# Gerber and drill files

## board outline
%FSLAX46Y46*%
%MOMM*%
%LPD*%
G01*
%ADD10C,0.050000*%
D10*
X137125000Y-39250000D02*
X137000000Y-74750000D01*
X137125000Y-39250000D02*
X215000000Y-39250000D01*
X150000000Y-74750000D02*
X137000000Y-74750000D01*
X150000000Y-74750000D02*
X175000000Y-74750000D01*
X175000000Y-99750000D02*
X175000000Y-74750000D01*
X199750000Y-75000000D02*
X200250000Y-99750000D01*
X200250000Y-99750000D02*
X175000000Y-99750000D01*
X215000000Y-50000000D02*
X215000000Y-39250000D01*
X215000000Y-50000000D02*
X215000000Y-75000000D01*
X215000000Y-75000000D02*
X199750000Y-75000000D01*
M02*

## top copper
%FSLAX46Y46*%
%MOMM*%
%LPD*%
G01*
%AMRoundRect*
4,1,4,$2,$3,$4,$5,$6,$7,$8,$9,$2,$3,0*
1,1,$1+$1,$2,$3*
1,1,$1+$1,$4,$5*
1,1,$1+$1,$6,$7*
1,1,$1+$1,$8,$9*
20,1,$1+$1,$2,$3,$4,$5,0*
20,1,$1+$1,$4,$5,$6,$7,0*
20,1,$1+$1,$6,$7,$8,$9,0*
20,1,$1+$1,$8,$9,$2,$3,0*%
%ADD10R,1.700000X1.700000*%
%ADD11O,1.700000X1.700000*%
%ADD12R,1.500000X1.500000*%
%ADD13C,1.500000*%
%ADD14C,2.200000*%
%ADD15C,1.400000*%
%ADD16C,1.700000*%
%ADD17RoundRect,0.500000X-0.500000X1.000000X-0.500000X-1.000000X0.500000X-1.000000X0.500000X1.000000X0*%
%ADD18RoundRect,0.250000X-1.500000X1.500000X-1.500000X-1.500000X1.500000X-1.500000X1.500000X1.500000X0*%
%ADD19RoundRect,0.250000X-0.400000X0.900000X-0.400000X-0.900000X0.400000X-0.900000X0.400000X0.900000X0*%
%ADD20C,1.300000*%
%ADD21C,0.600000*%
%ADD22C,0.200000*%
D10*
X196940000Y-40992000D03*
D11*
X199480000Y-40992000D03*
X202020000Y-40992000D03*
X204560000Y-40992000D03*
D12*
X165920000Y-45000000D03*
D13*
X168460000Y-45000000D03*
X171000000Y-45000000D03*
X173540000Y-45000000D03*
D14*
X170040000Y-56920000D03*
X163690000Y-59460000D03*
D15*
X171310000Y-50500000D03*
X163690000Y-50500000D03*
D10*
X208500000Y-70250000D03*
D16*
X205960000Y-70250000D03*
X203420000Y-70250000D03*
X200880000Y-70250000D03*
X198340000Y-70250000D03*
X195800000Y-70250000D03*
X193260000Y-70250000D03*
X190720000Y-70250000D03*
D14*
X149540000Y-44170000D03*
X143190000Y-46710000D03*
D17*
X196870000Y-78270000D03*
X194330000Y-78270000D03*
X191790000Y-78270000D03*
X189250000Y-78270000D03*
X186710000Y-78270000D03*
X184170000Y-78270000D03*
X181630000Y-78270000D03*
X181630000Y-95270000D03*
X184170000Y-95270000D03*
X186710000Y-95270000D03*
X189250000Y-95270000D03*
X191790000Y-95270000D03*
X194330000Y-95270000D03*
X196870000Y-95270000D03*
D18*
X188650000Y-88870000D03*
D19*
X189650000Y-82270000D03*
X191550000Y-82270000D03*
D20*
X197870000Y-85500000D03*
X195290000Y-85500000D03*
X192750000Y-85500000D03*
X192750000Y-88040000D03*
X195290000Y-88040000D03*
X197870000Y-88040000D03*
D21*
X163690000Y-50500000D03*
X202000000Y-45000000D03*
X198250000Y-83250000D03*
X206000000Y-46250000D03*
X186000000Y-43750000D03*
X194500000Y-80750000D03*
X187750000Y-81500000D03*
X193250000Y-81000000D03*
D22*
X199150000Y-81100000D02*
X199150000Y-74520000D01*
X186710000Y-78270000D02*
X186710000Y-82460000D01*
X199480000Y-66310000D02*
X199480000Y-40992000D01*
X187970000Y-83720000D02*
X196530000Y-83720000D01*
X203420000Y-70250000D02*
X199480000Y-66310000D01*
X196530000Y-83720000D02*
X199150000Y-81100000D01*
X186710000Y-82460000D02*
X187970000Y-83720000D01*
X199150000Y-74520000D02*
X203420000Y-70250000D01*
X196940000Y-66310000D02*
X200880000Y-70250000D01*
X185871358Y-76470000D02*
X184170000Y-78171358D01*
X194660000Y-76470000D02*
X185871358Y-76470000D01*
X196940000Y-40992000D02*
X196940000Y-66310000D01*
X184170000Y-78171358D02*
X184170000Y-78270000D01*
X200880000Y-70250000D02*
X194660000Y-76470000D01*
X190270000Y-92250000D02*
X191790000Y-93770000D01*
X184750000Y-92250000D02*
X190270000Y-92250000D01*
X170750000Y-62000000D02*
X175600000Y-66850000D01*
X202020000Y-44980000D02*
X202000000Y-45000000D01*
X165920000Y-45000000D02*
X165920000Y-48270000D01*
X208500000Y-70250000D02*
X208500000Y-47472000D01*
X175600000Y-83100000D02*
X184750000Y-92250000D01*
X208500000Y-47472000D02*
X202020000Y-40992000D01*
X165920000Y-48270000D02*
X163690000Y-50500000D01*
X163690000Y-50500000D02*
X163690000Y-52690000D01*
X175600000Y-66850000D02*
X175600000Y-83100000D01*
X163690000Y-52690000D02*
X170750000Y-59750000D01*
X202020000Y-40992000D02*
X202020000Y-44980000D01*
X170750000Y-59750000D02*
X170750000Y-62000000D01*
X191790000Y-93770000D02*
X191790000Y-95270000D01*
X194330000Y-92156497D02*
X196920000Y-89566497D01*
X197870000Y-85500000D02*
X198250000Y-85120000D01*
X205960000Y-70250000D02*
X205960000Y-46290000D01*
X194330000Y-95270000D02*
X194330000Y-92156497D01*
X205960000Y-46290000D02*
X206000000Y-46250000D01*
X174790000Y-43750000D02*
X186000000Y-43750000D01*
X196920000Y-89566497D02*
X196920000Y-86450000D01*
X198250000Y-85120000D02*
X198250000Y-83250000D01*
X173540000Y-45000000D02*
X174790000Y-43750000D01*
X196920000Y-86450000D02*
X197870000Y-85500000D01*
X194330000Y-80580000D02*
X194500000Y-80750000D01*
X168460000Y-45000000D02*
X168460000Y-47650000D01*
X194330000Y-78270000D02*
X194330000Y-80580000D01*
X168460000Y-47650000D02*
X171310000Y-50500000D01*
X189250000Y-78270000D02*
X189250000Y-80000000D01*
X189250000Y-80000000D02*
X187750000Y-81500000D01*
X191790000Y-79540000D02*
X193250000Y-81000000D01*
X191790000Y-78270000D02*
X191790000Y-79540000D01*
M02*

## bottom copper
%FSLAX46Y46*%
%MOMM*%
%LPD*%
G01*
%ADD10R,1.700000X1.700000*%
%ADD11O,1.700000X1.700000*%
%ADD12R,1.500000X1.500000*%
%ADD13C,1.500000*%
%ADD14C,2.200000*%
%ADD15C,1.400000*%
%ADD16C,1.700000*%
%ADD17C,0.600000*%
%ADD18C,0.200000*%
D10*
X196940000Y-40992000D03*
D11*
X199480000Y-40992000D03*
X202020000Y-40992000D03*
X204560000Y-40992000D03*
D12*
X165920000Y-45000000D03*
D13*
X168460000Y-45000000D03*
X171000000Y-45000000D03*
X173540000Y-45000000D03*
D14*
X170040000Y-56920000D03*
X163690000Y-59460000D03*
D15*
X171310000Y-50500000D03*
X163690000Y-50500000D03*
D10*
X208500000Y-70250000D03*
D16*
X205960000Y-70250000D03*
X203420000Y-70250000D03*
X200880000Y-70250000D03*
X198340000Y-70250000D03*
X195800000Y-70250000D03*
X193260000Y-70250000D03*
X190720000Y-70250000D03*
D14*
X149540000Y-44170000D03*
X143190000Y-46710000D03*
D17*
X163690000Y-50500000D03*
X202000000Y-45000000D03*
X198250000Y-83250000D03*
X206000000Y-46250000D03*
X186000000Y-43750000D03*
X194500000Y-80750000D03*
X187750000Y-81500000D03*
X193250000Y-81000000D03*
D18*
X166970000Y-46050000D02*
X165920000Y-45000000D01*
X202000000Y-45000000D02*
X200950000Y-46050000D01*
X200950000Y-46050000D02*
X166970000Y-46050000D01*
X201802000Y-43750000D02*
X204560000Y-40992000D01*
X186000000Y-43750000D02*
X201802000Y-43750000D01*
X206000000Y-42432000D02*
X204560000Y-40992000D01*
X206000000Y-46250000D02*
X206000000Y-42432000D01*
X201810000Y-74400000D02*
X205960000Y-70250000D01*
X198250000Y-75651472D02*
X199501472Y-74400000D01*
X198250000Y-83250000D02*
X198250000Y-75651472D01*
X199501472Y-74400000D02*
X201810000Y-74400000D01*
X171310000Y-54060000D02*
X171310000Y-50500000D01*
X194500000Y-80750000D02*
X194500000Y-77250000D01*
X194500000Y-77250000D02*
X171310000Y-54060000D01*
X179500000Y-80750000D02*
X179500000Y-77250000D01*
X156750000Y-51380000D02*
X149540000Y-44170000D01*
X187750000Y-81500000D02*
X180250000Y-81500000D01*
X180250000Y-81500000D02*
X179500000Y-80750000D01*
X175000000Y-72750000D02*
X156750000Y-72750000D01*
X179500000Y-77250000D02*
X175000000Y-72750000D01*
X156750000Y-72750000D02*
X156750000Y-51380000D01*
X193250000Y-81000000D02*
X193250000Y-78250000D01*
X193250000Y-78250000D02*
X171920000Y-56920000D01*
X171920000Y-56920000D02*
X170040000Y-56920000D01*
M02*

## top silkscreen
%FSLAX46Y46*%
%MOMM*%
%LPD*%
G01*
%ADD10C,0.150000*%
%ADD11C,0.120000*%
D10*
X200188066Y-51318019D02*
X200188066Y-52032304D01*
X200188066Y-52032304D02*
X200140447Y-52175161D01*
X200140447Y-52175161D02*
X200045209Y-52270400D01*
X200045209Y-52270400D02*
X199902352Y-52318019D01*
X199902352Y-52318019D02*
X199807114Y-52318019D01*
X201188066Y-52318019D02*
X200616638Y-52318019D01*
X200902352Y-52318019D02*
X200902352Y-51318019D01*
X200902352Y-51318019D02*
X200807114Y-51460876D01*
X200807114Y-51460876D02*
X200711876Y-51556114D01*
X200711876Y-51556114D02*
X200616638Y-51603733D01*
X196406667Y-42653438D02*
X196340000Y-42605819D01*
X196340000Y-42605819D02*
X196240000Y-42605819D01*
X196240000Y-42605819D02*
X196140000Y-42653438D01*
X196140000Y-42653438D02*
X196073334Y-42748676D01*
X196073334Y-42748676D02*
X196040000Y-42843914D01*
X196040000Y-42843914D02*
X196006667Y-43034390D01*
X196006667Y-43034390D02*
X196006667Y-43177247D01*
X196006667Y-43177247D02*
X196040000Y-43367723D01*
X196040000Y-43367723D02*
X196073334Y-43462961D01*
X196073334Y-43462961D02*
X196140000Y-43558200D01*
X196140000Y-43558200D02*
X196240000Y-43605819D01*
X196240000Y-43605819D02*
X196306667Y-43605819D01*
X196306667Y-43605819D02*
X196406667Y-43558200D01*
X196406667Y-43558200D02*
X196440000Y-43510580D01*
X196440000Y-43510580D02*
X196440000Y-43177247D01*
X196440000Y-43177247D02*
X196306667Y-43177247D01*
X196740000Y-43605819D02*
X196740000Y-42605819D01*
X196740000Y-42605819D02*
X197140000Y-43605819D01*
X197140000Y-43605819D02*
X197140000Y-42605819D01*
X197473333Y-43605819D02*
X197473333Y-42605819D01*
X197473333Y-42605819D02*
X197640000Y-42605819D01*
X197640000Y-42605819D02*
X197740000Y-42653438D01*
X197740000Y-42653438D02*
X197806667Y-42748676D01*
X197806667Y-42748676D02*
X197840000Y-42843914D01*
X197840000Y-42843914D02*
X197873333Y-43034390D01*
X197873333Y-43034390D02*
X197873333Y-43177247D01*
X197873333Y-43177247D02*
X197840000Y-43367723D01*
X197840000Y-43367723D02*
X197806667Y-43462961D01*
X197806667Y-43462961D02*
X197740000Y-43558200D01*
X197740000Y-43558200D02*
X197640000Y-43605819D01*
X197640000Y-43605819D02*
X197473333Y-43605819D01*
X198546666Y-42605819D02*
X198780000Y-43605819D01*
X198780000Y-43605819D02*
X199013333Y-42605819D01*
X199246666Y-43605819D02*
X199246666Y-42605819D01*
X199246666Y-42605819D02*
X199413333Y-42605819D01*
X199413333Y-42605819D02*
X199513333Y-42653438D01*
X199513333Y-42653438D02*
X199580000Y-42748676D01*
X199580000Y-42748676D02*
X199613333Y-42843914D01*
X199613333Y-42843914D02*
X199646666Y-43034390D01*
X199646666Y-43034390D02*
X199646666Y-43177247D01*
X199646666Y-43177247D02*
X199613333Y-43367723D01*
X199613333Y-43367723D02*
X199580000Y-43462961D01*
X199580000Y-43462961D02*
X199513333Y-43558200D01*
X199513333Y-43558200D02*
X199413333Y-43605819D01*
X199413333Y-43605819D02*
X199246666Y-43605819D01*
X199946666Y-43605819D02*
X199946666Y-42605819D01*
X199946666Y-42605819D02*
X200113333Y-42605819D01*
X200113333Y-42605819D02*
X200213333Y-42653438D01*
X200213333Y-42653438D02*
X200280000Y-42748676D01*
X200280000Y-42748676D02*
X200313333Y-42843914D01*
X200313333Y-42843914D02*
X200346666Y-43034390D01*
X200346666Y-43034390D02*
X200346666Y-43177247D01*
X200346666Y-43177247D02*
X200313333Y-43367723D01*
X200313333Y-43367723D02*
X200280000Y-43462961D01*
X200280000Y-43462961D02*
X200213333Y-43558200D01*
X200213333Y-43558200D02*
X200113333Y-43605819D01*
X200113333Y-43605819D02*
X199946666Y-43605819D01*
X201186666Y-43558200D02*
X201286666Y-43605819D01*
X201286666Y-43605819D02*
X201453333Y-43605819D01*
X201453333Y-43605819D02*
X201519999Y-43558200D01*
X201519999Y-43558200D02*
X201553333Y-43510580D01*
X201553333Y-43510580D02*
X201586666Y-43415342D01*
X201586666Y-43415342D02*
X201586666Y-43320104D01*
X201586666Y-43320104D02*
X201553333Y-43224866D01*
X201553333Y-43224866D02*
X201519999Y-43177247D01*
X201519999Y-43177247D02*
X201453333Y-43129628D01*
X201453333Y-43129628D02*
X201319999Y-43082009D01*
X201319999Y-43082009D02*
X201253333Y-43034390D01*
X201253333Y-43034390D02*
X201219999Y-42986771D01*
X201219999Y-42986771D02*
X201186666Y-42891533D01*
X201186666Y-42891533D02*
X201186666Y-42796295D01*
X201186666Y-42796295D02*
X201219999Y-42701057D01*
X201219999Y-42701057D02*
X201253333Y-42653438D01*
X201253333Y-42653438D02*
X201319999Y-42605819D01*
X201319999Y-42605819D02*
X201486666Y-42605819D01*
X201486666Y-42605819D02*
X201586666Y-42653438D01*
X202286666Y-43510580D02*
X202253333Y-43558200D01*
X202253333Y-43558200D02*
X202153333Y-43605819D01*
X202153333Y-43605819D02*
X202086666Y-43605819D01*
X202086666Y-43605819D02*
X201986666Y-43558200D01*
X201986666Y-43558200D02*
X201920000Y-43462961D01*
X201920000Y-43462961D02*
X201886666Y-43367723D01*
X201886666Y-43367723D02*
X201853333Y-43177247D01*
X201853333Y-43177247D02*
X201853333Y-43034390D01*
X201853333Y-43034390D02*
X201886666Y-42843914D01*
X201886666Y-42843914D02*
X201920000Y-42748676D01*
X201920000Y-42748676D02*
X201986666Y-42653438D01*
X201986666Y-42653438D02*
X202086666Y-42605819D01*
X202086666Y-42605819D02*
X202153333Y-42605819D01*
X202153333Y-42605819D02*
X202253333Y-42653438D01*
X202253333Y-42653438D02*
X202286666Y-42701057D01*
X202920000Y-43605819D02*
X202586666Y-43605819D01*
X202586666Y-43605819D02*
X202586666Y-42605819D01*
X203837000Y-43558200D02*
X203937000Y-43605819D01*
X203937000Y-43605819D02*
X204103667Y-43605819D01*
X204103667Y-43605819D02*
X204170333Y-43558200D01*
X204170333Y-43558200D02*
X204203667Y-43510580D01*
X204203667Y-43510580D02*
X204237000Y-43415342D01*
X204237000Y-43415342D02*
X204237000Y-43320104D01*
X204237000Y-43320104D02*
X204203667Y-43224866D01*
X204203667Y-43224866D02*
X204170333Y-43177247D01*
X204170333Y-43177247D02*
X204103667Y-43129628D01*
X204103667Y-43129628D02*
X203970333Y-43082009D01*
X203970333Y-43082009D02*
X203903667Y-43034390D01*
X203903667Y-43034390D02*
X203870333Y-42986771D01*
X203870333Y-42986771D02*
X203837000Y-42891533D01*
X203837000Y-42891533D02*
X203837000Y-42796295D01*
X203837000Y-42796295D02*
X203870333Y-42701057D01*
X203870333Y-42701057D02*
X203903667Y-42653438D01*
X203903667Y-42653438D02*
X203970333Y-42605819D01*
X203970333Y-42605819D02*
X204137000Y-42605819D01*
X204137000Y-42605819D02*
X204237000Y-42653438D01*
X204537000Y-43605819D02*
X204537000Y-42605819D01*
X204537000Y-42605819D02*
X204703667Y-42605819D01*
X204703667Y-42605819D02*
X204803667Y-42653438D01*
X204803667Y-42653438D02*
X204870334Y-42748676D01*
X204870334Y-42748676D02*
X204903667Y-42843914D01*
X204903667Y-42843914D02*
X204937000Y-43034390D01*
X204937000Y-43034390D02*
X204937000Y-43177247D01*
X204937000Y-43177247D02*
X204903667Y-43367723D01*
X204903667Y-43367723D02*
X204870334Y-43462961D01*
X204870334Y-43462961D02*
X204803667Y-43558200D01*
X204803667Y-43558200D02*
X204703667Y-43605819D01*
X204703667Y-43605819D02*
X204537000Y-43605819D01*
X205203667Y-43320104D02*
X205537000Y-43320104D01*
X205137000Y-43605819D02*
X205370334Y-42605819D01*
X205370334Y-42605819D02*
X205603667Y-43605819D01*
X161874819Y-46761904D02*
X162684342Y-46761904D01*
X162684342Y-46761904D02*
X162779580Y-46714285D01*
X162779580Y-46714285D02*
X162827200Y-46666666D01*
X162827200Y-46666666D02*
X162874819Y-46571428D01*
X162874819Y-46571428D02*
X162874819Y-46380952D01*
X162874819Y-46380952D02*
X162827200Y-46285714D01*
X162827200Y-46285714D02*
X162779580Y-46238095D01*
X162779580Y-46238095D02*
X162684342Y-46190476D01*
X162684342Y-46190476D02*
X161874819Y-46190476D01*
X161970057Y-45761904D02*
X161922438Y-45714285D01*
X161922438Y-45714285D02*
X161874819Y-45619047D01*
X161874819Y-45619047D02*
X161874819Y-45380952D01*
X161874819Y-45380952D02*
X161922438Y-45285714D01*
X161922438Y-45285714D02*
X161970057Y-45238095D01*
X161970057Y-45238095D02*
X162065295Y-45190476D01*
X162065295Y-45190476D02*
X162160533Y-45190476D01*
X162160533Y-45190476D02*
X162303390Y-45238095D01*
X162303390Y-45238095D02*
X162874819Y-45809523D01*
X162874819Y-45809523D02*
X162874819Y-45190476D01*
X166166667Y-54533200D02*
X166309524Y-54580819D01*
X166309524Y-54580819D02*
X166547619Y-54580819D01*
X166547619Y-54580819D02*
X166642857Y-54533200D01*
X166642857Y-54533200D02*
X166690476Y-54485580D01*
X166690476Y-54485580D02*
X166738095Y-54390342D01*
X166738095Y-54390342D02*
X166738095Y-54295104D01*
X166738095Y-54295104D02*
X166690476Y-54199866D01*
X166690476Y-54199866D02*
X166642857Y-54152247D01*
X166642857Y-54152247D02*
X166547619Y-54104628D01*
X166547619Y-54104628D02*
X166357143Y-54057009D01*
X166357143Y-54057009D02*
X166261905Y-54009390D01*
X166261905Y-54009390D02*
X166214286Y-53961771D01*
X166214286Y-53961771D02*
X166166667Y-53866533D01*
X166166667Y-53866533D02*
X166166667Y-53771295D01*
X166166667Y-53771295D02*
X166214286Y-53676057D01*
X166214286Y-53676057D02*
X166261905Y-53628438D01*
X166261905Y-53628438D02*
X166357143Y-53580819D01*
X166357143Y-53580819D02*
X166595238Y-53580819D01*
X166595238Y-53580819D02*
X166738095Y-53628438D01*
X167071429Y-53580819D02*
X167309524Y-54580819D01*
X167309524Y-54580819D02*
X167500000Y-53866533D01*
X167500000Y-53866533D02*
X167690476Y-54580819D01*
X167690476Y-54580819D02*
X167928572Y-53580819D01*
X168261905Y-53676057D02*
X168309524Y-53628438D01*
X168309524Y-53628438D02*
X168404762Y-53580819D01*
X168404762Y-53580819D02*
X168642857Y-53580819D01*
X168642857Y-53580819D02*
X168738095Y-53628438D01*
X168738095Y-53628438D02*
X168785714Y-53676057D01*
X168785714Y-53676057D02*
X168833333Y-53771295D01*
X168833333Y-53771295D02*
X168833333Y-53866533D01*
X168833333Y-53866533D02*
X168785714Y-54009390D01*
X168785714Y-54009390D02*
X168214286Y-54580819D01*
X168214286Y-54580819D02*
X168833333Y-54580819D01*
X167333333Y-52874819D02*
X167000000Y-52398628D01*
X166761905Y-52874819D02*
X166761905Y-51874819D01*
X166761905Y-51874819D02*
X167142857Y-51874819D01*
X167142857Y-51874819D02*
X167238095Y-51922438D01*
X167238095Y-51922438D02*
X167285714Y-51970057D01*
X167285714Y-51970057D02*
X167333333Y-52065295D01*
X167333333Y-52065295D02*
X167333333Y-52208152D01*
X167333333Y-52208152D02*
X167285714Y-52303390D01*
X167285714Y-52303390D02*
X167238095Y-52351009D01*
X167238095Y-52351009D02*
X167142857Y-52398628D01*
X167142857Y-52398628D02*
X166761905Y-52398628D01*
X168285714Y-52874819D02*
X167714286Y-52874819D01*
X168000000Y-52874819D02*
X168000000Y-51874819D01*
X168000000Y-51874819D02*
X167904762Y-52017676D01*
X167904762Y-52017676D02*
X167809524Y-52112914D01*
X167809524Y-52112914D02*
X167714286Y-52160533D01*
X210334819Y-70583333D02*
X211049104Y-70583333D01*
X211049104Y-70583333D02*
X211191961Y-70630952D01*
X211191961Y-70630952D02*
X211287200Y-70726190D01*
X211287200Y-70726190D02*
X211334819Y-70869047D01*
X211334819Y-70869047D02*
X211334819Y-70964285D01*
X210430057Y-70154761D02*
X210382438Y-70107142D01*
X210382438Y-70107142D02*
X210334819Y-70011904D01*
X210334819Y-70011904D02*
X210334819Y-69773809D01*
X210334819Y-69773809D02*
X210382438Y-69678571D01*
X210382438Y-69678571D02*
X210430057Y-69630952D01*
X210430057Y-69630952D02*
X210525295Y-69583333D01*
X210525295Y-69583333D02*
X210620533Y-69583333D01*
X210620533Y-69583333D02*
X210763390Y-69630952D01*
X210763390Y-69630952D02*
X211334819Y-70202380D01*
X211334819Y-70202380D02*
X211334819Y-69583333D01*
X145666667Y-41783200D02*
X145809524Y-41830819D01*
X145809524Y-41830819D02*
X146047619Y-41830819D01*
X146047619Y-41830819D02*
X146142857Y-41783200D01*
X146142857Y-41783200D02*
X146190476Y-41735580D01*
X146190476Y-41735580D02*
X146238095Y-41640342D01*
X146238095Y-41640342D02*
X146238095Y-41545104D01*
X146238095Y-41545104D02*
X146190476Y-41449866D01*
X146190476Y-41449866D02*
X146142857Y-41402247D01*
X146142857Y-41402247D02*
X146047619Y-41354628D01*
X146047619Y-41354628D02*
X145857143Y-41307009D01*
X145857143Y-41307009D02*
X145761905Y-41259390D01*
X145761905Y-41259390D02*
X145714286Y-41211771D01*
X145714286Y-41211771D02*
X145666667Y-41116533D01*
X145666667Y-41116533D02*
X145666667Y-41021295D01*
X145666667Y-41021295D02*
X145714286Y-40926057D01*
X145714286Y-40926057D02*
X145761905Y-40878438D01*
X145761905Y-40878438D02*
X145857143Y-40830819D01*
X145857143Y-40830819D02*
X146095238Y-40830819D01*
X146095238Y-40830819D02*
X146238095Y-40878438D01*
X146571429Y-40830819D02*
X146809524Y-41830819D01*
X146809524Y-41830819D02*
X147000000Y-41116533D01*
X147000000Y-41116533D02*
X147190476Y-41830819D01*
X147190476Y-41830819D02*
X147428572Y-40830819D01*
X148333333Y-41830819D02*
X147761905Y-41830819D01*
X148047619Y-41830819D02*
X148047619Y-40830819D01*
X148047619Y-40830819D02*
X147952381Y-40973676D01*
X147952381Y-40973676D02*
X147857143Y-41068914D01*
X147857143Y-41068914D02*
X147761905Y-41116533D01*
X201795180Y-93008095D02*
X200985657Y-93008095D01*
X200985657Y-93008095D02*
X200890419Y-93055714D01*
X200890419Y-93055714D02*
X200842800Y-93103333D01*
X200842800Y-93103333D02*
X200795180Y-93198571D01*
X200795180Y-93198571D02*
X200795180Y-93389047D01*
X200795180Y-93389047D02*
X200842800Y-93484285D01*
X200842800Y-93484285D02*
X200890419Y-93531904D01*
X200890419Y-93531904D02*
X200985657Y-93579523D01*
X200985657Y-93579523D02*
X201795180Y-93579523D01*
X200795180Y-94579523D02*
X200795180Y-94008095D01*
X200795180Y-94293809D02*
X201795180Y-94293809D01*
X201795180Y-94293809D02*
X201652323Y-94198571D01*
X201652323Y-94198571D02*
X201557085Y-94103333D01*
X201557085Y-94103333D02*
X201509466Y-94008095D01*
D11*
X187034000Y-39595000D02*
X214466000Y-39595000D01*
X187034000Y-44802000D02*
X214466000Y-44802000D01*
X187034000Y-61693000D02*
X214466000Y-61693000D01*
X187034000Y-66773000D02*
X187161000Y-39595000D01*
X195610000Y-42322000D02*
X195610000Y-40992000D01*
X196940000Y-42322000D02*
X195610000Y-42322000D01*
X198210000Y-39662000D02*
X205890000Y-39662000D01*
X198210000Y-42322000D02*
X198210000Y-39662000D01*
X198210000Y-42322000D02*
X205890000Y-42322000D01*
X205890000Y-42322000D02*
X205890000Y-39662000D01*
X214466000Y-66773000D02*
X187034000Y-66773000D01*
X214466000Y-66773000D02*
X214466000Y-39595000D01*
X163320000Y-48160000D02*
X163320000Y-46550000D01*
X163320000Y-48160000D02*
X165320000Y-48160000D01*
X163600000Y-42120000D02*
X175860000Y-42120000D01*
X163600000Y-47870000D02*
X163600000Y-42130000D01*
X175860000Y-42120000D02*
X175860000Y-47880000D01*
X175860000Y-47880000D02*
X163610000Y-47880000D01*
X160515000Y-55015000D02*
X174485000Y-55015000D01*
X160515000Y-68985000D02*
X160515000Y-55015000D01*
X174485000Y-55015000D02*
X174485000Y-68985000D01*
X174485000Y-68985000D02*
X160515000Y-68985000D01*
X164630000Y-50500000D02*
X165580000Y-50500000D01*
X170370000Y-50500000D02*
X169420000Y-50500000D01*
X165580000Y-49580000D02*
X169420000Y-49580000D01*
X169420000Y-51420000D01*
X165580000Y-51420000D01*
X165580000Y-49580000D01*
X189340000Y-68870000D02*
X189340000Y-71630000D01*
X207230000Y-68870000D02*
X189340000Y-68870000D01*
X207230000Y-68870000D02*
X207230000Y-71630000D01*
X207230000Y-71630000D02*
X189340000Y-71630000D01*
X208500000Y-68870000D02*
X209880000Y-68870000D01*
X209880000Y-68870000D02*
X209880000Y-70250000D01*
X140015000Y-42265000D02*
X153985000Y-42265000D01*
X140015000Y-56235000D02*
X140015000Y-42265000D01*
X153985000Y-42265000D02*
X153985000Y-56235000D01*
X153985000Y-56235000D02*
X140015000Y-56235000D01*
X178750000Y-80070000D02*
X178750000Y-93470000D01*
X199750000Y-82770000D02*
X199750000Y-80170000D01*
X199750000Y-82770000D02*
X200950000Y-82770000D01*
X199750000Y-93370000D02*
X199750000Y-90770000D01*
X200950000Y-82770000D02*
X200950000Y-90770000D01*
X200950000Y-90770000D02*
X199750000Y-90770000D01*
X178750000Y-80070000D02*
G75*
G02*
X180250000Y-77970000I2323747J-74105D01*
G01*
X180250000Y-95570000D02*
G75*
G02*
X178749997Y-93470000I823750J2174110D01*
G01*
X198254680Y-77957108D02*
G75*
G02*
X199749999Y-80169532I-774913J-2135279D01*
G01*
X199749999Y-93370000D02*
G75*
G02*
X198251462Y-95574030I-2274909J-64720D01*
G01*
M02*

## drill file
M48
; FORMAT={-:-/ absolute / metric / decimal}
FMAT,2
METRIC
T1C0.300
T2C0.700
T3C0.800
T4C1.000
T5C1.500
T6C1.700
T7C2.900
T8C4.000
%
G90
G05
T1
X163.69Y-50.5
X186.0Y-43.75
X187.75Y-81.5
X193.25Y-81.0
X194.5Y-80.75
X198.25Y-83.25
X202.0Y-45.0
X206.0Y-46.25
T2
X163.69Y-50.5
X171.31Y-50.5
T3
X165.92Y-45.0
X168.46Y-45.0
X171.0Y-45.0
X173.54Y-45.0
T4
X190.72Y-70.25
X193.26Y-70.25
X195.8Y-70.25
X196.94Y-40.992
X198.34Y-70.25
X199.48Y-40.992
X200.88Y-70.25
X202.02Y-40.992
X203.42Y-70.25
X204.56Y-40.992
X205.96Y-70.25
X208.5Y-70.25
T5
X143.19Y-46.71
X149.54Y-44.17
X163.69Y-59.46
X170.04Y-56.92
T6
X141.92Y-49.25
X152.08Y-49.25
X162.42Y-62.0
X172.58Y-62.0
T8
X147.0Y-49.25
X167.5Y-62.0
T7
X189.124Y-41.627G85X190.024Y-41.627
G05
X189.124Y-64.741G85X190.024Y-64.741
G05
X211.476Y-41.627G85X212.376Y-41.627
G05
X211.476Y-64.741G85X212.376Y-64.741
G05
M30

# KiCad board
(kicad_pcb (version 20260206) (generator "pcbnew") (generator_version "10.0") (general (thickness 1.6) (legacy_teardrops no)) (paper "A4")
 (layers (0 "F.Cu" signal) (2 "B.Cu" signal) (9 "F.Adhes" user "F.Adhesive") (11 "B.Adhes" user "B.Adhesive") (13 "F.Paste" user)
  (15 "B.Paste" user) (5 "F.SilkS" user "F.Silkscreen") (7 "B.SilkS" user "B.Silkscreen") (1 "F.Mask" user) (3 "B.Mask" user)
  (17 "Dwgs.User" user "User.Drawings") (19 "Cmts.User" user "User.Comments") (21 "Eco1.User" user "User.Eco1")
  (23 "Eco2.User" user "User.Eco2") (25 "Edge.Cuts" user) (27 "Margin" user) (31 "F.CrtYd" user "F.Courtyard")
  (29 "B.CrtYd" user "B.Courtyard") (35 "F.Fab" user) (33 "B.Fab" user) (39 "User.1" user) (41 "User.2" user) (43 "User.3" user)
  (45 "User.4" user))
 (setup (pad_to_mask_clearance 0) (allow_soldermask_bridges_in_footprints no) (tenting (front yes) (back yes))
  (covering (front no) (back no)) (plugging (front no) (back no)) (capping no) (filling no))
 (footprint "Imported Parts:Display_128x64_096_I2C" (layer "F.Cu") (at 200.75 40.992)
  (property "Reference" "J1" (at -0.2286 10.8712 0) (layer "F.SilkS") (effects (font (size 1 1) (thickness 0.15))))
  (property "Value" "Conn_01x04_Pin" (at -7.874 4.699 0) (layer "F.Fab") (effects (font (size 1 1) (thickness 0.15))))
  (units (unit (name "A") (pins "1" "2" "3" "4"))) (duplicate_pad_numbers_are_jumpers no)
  (fp_line (start -13.716 -1.397) (end 13.716 -1.397) (stroke (width 0.12) (type solid)) (layer "F.SilkS"))
  (fp_line (start -13.716 3.81) (end 13.716 3.81) (stroke (width 0.12) (type solid)) (layer "F.SilkS"))
  (fp_line (start -13.716 20.701) (end 13.716 20.701) (stroke (width 0.12) (type solid)) (layer "F.SilkS"))
  (fp_line (start -13.716 25.781) (end -13.589 -1.397) (stroke (width 0.12) (type solid)) (layer "F.SilkS"))
  (fp_line (start -5.14 1.33) (end -5.14 0) (stroke (width 0.12) (type solid)) (layer "F.SilkS"))
  (fp_line (start -3.81 1.33) (end -5.14 1.33) (stroke (width 0.12) (type solid)) (layer "F.SilkS"))
  (fp_line (start -2.54 -1.33) (end 5.14 -1.33) (stroke (width 0.12) (type solid)) (layer "F.SilkS"))
  (fp_line (start -2.54 1.33) (end -2.54 -1.33) (stroke (width 0.12) (type solid)) (layer "F.SilkS"))
  (fp_line (start -2.54 1.33) (end 5.14 1.33) (stroke (width 0.12) (type solid)) (layer "F.SilkS"))
  (fp_line (start 5.14 1.33) (end 5.14 -1.33) (stroke (width 0.12) (type solid)) (layer "F.SilkS"))
  (fp_line (start 13.716 25.781) (end -13.716 25.781) (stroke (width 0.12) (type solid)) (layer "F.SilkS"))
  (fp_line (start 13.716 25.781) (end 13.716 -1.397) (stroke (width 0.12) (type solid)) (layer "F.SilkS"))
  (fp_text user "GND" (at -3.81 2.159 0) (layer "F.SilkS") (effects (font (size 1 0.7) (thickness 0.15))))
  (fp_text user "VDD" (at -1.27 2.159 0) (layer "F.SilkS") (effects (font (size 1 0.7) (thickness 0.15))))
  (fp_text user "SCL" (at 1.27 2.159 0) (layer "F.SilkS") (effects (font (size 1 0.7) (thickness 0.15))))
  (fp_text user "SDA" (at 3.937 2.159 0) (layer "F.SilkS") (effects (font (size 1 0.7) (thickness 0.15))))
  (pad "" np_thru_hole oval (at -11.176 0.635) (size 3.8 2.9) (drill oval 3.8 2.9) (layers "*.Cu" "*.Mask"))
  (pad "" np_thru_hole oval (at -11.176 23.749) (size 3.8 2.9) (drill oval 3.8 2.9) (layers "*.Cu" "*.Mask"))
  (pad "" np_thru_hole oval (at 11.176 0.635) (size 3.8 2.9) (drill oval 3.8 2.9) (layers "*.Cu" "*.Mask"))
  (pad "" np_thru_hole oval (at 11.176 23.749) (size 3.8 2.9) (drill oval 3.8 2.9) (layers "*.Cu" "*.Mask"))
  (pad "1" thru_hole rect (at -3.81 0 90) (size 1.7 1.7) (drill 1) (layers "*.Cu" "*.Mask") (remove_unused_layers no) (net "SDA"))
  (pad "2" thru_hole oval (at -1.27 0 90) (size 1.7 1.7) (drill 1) (layers "*.Cu" "*.Mask") (remove_unused_layers no) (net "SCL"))
  (pad "3" thru_hole oval (at 1.27 0 90) (size 1.7 1.7) (drill 1) (layers "*.Cu" "*.Mask") (remove_unused_layers no) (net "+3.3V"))
  (pad "4" thru_hole oval (at 3.81 0 90) (size 1.7 1.7) (drill 1) (layers "*.Cu" "*.Mask") (remove_unused_layers no) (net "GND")))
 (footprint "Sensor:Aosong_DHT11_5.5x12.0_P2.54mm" (layer "F.Cu") (at 165.92 45 90)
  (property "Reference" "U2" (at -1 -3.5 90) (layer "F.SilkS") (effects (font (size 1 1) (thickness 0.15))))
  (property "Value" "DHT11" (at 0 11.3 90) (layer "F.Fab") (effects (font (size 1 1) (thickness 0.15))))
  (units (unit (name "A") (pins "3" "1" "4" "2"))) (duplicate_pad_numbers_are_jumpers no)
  (fp_line (start -3.16 -2.6) (end -1.55 -2.6) (stroke (width 0.12) (type solid)) (layer "F.SilkS"))
  (fp_line (start -3.16 -2.6) (end -3.16 -0.6) (stroke (width 0.12) (type solid)) (layer "F.SilkS"))
  (fp_line (start 2.88 -2.32) (end 2.88 9.94) (stroke (width 0.12) (type solid)) (layer "F.SilkS"))
  (fp_line (start -2.87 -2.32) (end 2.87 -2.32) (stroke (width 0.12) (type solid)) (layer "F.SilkS"))
  (fp_line (start 2.88 9.94) (end -2.88 9.94) (stroke (width 0.12) (type solid)) (layer "F.SilkS"))
  (fp_line (start -2.88 9.94) (end -2.88 -2.31) (stroke (width 0.12) (type solid)) (layer "F.SilkS"))
  (pad "1" thru_hole rect (at 0 0 90) (size 1.5 1.5) (drill 0.8) (layers "*.Cu" "*.Mask") (remove_unused_layers no) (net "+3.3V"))
  (pad "2" thru_hole circle (at 0 2.54 90) (size 1.5 1.5) (drill 0.8) (layers "*.Cu" "*.Mask") (remove_unused_layers no) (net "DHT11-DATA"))
  (pad "3" thru_hole circle (at 0 5.08 90) (size 1.5 1.5) (drill 0.8) (layers "*.Cu" "*.Mask") (remove_unused_layers no)
   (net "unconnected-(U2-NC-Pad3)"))
  (pad "4" thru_hole circle (at 0 7.62 90) (size 1.5 1.5) (drill 0.8) (layers "*.Cu" "*.Mask") (remove_unused_layers no) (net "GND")))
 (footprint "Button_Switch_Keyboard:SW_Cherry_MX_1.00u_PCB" (layer "F.Cu") (at 170.04 56.92)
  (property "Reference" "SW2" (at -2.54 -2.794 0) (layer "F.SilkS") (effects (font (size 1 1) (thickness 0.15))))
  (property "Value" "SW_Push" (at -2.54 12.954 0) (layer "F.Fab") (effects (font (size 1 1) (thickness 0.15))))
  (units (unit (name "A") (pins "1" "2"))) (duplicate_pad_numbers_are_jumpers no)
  (fp_line (start -9.525 -1.905) (end 4.445 -1.905) (stroke (width 0.12) (type solid)) (layer "F.SilkS"))
  (fp_line (start -9.525 12.065) (end -9.525 -1.905) (stroke (width 0.12) (type solid)) (layer "F.SilkS"))
  (fp_line (start 4.445 -1.905) (end 4.445 12.065) (stroke (width 0.12) (type solid)) (layer "F.SilkS"))
  (fp_line (start 4.445 12.065) (end -9.525 12.065) (stroke (width 0.12) (type solid)) (layer "F.SilkS"))
  (pad "" np_thru_hole circle (at -7.62 5.08) (size 1.7 1.7) (drill 1.7) (layers "*.Cu" "*.Mask"))
  (pad "" np_thru_hole circle (at -2.54 5.08) (size 4 4) (drill 4) (layers "*.Cu" "*.Mask"))
  (pad "" np_thru_hole circle (at 2.54 5.08) (size 1.7 1.7) (drill 1.7) (layers "*.Cu" "*.Mask"))
  (pad "1" thru_hole circle (at 0 0) (size 2.2 2.2) (drill 1.5) (layers "*.Cu" "*.Mask") (remove_unused_layers no) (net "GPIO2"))
  (pad "2" thru_hole circle (at -6.35 2.54) (size 2.2 2.2) (drill 1.5) (layers "*.Cu" "*.Mask") (remove_unused_layers no) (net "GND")))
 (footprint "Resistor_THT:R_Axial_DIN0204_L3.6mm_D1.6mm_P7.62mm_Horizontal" (layer "F.Cu") (at 171.31 50.5 180)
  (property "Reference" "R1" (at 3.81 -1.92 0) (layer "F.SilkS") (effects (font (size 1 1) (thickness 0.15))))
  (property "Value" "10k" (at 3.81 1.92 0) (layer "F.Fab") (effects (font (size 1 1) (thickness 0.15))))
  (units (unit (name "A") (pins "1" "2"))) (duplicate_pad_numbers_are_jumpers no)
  (fp_line (start 6.68 0) (end 5.73 0) (stroke (width 0.12) (type solid)) (layer "F.SilkS"))
  (fp_line (start 0.94 0) (end 1.89 0) (stroke (width 0.12) (type solid)) (layer "F.SilkS"))
  (fp_rect (start 1.89 -0.92) (end 5.73 0.92) (stroke (width 0.12) (type solid)) (fill no) (layer "F.SilkS"))
  (pad "1" thru_hole circle (at 0 0 180) (size 1.4 1.4) (drill 0.7) (layers "*.Cu" "*.Mask") (remove_unused_layers no) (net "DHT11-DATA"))
  (pad "2" thru_hole circle (at 7.62 0 180) (size 1.4 1.4) (drill 0.7) (layers "*.Cu" "*.Mask") (remove_unused_layers no) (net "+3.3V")))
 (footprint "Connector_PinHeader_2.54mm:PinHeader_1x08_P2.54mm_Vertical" (layer "F.Cu") (at 208.5 70.25 -90)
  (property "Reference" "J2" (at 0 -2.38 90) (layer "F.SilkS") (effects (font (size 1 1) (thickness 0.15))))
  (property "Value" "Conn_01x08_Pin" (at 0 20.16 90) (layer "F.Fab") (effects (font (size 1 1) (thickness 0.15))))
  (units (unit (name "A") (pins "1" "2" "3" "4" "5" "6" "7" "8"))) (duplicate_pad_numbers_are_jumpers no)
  (fp_line (start -1.38 19.16) (end 1.38 19.16) (stroke (width 0.12) (type solid)) (layer "F.SilkS"))
  (fp_line (start -1.38 1.27) (end -1.38 19.16) (stroke (width 0.12) (type solid)) (layer "F.SilkS"))
  (fp_line (start -1.38 1.27) (end 1.38 1.27) (stroke (width 0.12) (type solid)) (layer "F.SilkS"))
  (fp_line (start 1.38 1.27) (end 1.38 19.16) (stroke (width 0.12) (type solid)) (layer "F.SilkS"))
  (fp_line (start -1.38 0) (end -1.38 -1.38) (stroke (width 0.12) (type solid)) (layer "F.SilkS"))
  (fp_line (start -1.38 -1.38) (end 0 -1.38) (stroke (width 0.12) (type solid)) (layer "F.SilkS"))
  (pad "1" thru_hole rect (at 0 0 270) (size 1.7 1.7) (drill 1) (layers "*.Cu" "*.Mask") (remove_unused_layers no) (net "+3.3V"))
  (pad "2" thru_hole circle (at 0 2.54 270) (size 1.7 1.7) (drill 1) (layers "*.Cu" "*.Mask") (remove_unused_layers no) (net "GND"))
  (pad "3" thru_hole circle (at 0 5.08 270) (size 1.7 1.7) (drill 1) (layers "*.Cu" "*.Mask") (remove_unused_layers no) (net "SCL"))
  (pad "4" thru_hole circle (at 0 7.62 270) (size 1.7 1.7) (drill 1) (layers "*.Cu" "*.Mask") (remove_unused_layers no) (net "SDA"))
  (pad "5" thru_hole circle (at 0 10.16 270) (size 1.7 1.7) (drill 1) (layers "*.Cu" "*.Mask") (remove_unused_layers no)
   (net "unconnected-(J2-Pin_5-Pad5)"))
  (pad "6" thru_hole circle (at 0 12.7 270) (size 1.7 1.7) (drill 1) (layers "*.Cu" "*.Mask") (remove_unused_layers no)
   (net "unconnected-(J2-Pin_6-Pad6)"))
  (pad "7" thru_hole circle (at 0 15.24 270) (size 1.7 1.7) (drill 1) (layers "*.Cu" "*.Mask") (remove_unused_layers no)
   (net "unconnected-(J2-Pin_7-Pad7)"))
  (pad "8" thru_hole circle (at 0 17.78 270) (size 1.7 1.7) (drill 1) (layers "*.Cu" "*.Mask") (remove_unused_layers no)
   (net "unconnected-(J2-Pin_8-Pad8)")))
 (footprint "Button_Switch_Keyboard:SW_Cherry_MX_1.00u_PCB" (layer "F.Cu") (at 149.54 44.17)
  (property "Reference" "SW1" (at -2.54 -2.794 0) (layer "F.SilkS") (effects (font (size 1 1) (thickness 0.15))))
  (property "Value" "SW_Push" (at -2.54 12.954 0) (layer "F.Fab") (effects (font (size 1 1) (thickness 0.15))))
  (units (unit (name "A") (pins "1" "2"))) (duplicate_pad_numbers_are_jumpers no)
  (fp_line (start -9.525 -1.905) (end 4.445 -1.905) (stroke (width 0.12) (type solid)) (layer "F.SilkS"))
  (fp_line (start -9.525 12.065) (end -9.525 -1.905) (stroke (width 0.12) (type solid)) (layer "F.SilkS"))
  (fp_line (start 4.445 -1.905) (end 4.445 12.065) (stroke (width 0.12) (type solid)) (layer "F.SilkS"))
  (fp_line (start 4.445 12.065) (end -9.525 12.065) (stroke (width 0.12) (type solid)) (layer "F.SilkS"))
  (pad "" np_thru_hole circle (at -7.62 5.08) (size 1.7 1.7) (drill 1.7) (layers "*.Cu" "*.Mask"))
  (pad "" np_thru_hole circle (at -2.54 5.08) (size 4 4) (drill 4) (layers "*.Cu" "*.Mask"))
  (pad "" np_thru_hole circle (at 2.54 5.08) (size 1.7 1.7) (drill 1.7) (layers "*.Cu" "*.Mask"))
  (pad "1" thru_hole circle (at 0 0) (size 2.2 2.2) (drill 1.5) (layers "*.Cu" "*.Mask") (remove_unused_layers no) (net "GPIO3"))
  (pad "2" thru_hole circle (at -6.35 2.54) (size 2.2 2.2) (drill 1.5) (layers "*.Cu" "*.Mask") (remove_unused_layers no) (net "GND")))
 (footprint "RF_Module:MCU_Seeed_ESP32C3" (layer "F.Cu") (at 189.25 86.77 -90)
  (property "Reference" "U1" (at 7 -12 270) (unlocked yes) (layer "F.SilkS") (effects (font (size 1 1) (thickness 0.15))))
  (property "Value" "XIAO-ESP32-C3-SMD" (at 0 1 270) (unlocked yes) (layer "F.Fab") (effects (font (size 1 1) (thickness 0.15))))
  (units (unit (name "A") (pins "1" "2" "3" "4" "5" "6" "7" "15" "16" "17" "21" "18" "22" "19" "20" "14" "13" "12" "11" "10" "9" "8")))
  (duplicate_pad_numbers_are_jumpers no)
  (fp_line (start -6.7 10.5) (end 6.7 10.5) (stroke (width 0.12) (type default)) (layer "F.SilkS"))
  (fp_line (start -4 -10.5) (end -6.6 -10.5) (stroke (width 0.12) (type default)) (layer "F.SilkS"))
  (fp_line (start -4 -10.5) (end -4 -11.7) (stroke (width 0.12) (type default)) (layer "F.SilkS"))
  (fp_line (start 6.6 -10.5) (end 4 -10.5) (stroke (width 0.12) (type default)) (layer "F.SilkS"))
  (fp_line (start -4 -11.7) (end 4 -11.7) (stroke (width 0.12) (type default)) (layer "F.SilkS"))
  (fp_line (start 4 -11.7) (end 4 -10.5) (stroke (width 0.12) (type default)) (layer "F.SilkS"))
  (fp_arc (start -6.7 10.5) (mid -7.977232 10.068125) (end -8.8 9) (stroke (width 0.12) (type default)) (layer "F.SilkS"))
  (fp_arc (start 8.8 9) (mid 7.977232 10.068125) (end 6.7 10.5) (stroke (width 0.12) (type default)) (layer "F.SilkS"))
  (fp_arc (start -8.812892 -9.00468) (mid -7.949609 -10.111769) (end -6.600468 -10.499999) (stroke (width 0.12) (type default))
   (layer "F.SilkS"))
  (fp_arc (start 6.6 -10.499999) (mid 7.944325 -10.107116) (end 8.804034 -9.001464) (stroke (width 0.12) (type default)) (layer "F.SilkS"))
  (pad "" smd roundrect (at 1.1 -0.4 270) (size 1.5 1.5) (layers "F.Paste") (roundrect_rratio 0.1666666667))
  (pad "" smd roundrect (at 1.1 1.6 270) (size 1.5 1.5) (layers "F.Paste") (roundrect_rratio 0.1666666667))
  (pad "" smd roundrect (at 3.1 -0.4 270) (size 1.5 1.5) (layers "F.Paste") (roundrect_rratio 0.1666666667))
  (pad "" smd roundrect (at 3.1 1.6 270) (size 1.5 1.5) (layers "F.Paste") (roundrect_rratio 0.1666666667))
  (pad "1" smd roundrect (at -8.5 -7.62 270) (size 3 2) (layers "F.Cu" "F.Mask" "F.Paste") (roundrect_rratio 0.25)
   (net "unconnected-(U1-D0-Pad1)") (thermal_bridge_angle 45))
  (pad "2" smd roundrect (at -8.5 -5.08 270) (size 3 2) (layers "F.Cu" "F.Mask" "F.Paste") (roundrect_rratio 0.25) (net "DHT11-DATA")
   (thermal_bridge_angle 45))
  (pad "3" smd roundrect (at -8.5 -2.54 270) (size 3 2) (layers "F.Cu" "F.Mask" "F.Paste") (roundrect_rratio 0.25) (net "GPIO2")
   (thermal_bridge_angle 45))
  (pad "4" smd roundrect (at -8.5 0 270) (size 3 2) (layers "F.Cu" "F.Mask" "F.Paste") (roundrect_rratio 0.25) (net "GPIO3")
   (thermal_bridge_angle 45))
  (pad "5" smd roundrect (at -8.5 2.54 270) (size 3 2) (layers "F.Cu" "F.Mask" "F.Paste") (roundrect_rratio 0.25) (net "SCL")
   (thermal_bridge_angle 45))
  (pad "6" smd roundrect (at -8.5 5.08 270) (size 3 2) (layers "F.Cu" "F.Mask" "F.Paste") (roundrect_rratio 0.25) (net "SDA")
   (thermal_bridge_angle 45))
  (pad "7" smd roundrect (at -8.5 7.62 270) (size 3 2) (layers "F.Cu" "F.Mask" "F.Paste") (roundrect_rratio 0.25)
   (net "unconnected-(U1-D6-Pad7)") (thermal_bridge_angle 45))
  (pad "8" smd roundrect (at 8.5 7.62 270) (size 3 2) (layers "F.Cu" "F.Mask" "F.Paste") (roundrect_rratio 0.25)
   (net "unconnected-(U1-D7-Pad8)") (thermal_bridge_angle 45))
  (pad "9" smd roundrect (at 8.5 5.08 270) (size 3 2) (layers "F.Cu" "F.Mask" "F.Paste") (roundrect_rratio 0.25)
   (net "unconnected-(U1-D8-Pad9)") (thermal_bridge_angle 45))
  (pad "10" smd roundrect (at 8.5 2.54 270) (size 3 2) (layers "F.Cu" "F.Mask" "F.Paste") (roundrect_rratio 0.25)
   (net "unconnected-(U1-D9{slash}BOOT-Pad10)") (thermal_bridge_angle 45))
  (pad "11" smd roundrect (at 8.5 0 270) (size 3 2) (layers "F.Cu" "F.Mask" "F.Paste") (roundrect_rratio 0.25)
   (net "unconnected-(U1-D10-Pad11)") (thermal_bridge_angle 45))
  (pad "12" smd roundrect (at 8.5 -2.54 270) (size 3 2) (layers "F.Cu" "F.Mask" "F.Paste") (roundrect_rratio 0.25) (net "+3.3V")
   (thermal_bridge_angle 45))
  (pad "13" smd roundrect (at 8.5 -5.08 270) (size 3 2) (layers "F.Cu" "F.Mask" "F.Paste") (roundrect_rratio 0.25) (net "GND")
   (thermal_bridge_angle 45))
  (pad "14" smd roundrect (at 8.5 -7.62 270) (size 3 2) (layers "F.Cu" "F.Mask" "F.Paste") (roundrect_rratio 0.25) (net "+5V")
   (thermal_bridge_angle 45))
  (pad "15" smd roundrect (at 2.1 0.6 270) (size 3.5 3.5) (layers "F.Cu" "F.Mask") (roundrect_rratio 0.07142857143)
   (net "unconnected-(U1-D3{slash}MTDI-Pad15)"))
  (pad "16" smd roundrect (at -4.5 -0.4 270) (size 2.3 1.3) (layers "F.Cu" "F.Mask" "F.Paste") (roundrect_rratio 0.1923076923)
   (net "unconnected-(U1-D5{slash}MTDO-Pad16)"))
  (pad "17" smd roundrect (at -4.5 -2.3 270) (size 2.3 1.3) (layers "F.Cu" "F.Mask" "F.Paste") (roundrect_rratio 0.1923076923)
   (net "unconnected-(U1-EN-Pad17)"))
  (pad "18" smd circle (at -1.27 -8.62 270) (size 1.3 1.3) (layers "F.Cu" "F.Mask" "F.Paste") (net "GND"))
  (pad "19" smd circle (at -1.27 -6.04 270) (size 1.3 1.3) (layers "F.Cu" "F.Mask" "F.Paste") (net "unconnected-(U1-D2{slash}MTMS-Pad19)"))
  (pad "20" smd circle (at -1.27 -3.5 270) (size 1.3 1.3) (layers "F.Cu" "F.Mask" "F.Paste") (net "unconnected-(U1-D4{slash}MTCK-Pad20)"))
  (pad "21" smd circle (at 1.27 -3.5 270) (size 1.3 1.3) (layers "F.Cu" "F.Mask" "F.Paste") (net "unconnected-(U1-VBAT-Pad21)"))
  (pad "22" smd circle (at 1.27 -6.04 270) (size 1.3 1.3) (layers "F.Cu" "F.Mask" "F.Paste") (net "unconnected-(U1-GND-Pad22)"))
  (pad "23" smd circle (at 1.27 -8.62 270) (size 1.3 1.3) (layers "F.Cu" "F.Mask" "F.Paste")))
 (gr_line (start 137.125 39.25) (end 137 74.75) (stroke (width 0.05) (type default)) (layer "Edge.Cuts"))
 (gr_line (start 137.125 39.25) (end 215 39.25) (stroke (width 0.05) (type default)) (layer "Edge.Cuts"))
 (gr_line (start 150 74.75) (end 137 74.75) (stroke (width 0.05) (type default)) (layer "Edge.Cuts"))
 (gr_line (start 150 74.75) (end 175 74.75) (stroke (width 0.05) (type default)) (layer "Edge.Cuts"))
 (gr_line (start 175 99.75) (end 175 74.75) (stroke (width 0.05) (type default)) (layer "Edge.Cuts"))
 (gr_line (start 199.75 75) (end 200.25 99.75) (stroke (width 0.05) (type default)) (layer "Edge.Cuts"))
 (gr_line (start 200.25 99.75) (end 175 99.75) (stroke (width 0.05) (type default)) (layer "Edge.Cuts"))
 (gr_line (start 215 50) (end 215 39.25) (stroke (width 0.05) (type default)) (layer "Edge.Cuts"))
 (gr_line (start 215 50) (end 215 75) (stroke (width 0.05) (type default)) (layer "Edge.Cuts"))
 (gr_line (start 215 75) (end 199.75 75) (stroke (width 0.05) (type default)) (layer "Edge.Cuts"))
 (segment (start 199.15 81.1) (end 199.15 74.52) (width 0.2) (layer "F.Cu") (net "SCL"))
 (segment (start 186.71 78.27) (end 186.71 82.46) (width 0.2) (layer "F.Cu") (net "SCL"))
 (segment (start 199.48 66.31) (end 199.48 40.992) (width 0.2) (layer "F.Cu") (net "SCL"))
 (segment (start 187.97 83.72) (end 196.53 83.72) (width 0.2) (layer "F.Cu") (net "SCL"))
 (segment (start 203.42 70.25) (end 199.48 66.31) (width 0.2) (layer "F.Cu") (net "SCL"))
 (segment (start 196.53 83.72) (end 199.15 81.1) (width 0.2) (layer "F.Cu") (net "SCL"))
 (segment (start 186.71 82.46) (end 187.97 83.72) (width 0.2) (layer "F.Cu") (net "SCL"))
 (segment (start 199.15 74.52) (end 203.42 70.25) (width 0.2) (layer "F.Cu") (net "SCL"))
 (segment (start 196.94 66.31) (end 200.88 70.25) (width 0.2) (layer "F.Cu") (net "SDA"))
 (segment (start 185.871358 76.47) (end 184.17 78.171358) (width 0.2) (layer "F.Cu") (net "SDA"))
 (segment (start 194.66 76.47) (end 185.871358 76.47) (width 0.2) (layer "F.Cu") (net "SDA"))
 (segment (start 196.94 40.992) (end 196.94 66.31) (width 0.2) (layer "F.Cu") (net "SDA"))
 (segment (start 184.17 78.171358) (end 184.17 78.27) (width 0.2) (layer "F.Cu") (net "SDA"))
 (segment (start 200.88 70.25) (end 194.66 76.47) (width 0.2) (layer "F.Cu") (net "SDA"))
 (segment (start 190.27 92.25) (end 191.79 93.77) (width 0.2) (layer "F.Cu") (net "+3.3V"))
 (segment (start 184.75 92.25) (end 190.27 92.25) (width 0.2) (layer "F.Cu") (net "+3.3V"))
 (segment (start 170.75 62) (end 175.6 66.85) (width 0.2) (layer "F.Cu") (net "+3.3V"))
 (segment (start 202.02 44.98) (end 202 45) (width 0.2) (layer "F.Cu") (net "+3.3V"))
 (segment (start 165.92 45) (end 165.92 48.27) (width 0.2) (layer "F.Cu") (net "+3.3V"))
 (segment (start 208.5 70.25) (end 208.5 47.472) (width 0.2) (layer "F.Cu") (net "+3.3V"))
 (segment (start 175.6 83.1) (end 184.75 92.25) (width 0.2) (layer "F.Cu") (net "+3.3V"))
 (segment (start 208.5 47.472) (end 202.02 40.992) (width 0.2) (layer "F.Cu") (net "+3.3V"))
 (segment (start 165.92 48.27) (end 163.69 50.5) (width 0.2) (layer "F.Cu") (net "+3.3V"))
 (segment (start 163.69 50.5) (end 163.69 52.69) (width 0.2) (layer "F.Cu") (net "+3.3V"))
 (segment (start 175.6 66.85) (end 175.6 83.1) (width 0.2) (layer "F.Cu") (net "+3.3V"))
 (segment (start 163.69 52.69) (end 170.75 59.75) (width 0.2) (layer "F.Cu") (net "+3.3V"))
 (segment (start 202.02 40.992) (end 202.02 44.98) (width 0.2) (layer "F.Cu") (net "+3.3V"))
 (segment (start 170.75 59.75) (end 170.75 62) (width 0.2) (layer "F.Cu") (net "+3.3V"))
 (segment (start 191.79 93.77) (end 191.79 95.27) (width 0.2) (layer "F.Cu") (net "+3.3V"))
 (via (at 163.69 50.5) (size 0.6) (drill 0.3) (layers "F.Cu" "B.Cu") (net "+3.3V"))
 (via (at 202 45) (size 0.6) (drill 0.3) (layers "F.Cu" "B.Cu") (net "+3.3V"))
 (segment (start 166.97 46.05) (end 165.92 45) (width 0.2) (layer "B.Cu") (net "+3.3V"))
 (segment (start 202 45) (end 200.95 46.05) (width 0.2) (layer "B.Cu") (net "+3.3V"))
 (segment (start 200.95 46.05) (end 166.97 46.05) (width 0.2) (layer "B.Cu") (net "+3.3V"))
 (segment (start 194.33 92.156497) (end 196.92 89.566497) (width 0.2) (layer "F.Cu") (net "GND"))
 (segment (start 197.87 85.5) (end 198.25 85.12) (width 0.2) (layer "F.Cu") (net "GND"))
 (segment (start 205.96 70.25) (end 205.96 46.29) (width 0.2) (layer "F.Cu") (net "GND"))
 (segment (start 194.33 95.27) (end 194.33 92.156497) (width 0.2) (layer "F.Cu") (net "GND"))
 (segment (start 205.96 46.29) (end 206 46.25) (width 0.2) (layer "F.Cu") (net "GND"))
 (segment (start 174.79 43.75) (end 186 43.75) (width 0.2) (layer "F.Cu") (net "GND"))
 (segment (start 196.92 89.566497) (end 196.92 86.45) (width 0.2) (layer "F.Cu") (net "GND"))
 (segment (start 198.25 85.12) (end 198.25 83.25) (width 0.2) (layer "F.Cu") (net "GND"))
 (segment (start 173.54 45) (end 174.79 43.75) (width 0.2) (layer "F.Cu") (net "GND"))
 (segment (start 196.92 86.45) (end 197.87 85.5) (width 0.2) (layer "F.Cu") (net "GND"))
 (via (at 198.25 83.25) (size 0.6) (drill 0.3) (layers "F.Cu" "B.Cu") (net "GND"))
 (via (at 206 46.25) (size 0.6) (drill 0.3) (layers "F.Cu" "B.Cu") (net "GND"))
 (via (at 186 43.75) (size 0.6) (drill 0.3) (layers "F.Cu" "B.Cu") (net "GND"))
 (segment (start 201.802 43.75) (end 204.56 40.992) (width 0.2) (layer "B.Cu") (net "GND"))
 (segment (start 186 43.75) (end 201.802 43.75) (width 0.2) (layer "B.Cu") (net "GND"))
 (segment (start 206 42.432) (end 204.56 40.992) (width 0.2) (layer "B.Cu") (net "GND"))
 (segment (start 206 46.25) (end 206 42.432) (width 0.2) (layer "B.Cu") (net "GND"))
 (segment (start 201.81 74.4) (end 205.96 70.25) (width 0.2) (layer "B.Cu") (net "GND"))
 (segment (start 198.25 75.651472) (end 199.501472 74.4) (width 0.2) (layer "B.Cu") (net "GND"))
 (segment (start 198.25 83.25) (end 198.25 75.651472) (width 0.2) (layer "B.Cu") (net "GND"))
 (segment (start 199.501472 74.4) (end 201.81 74.4) (width 0.2) (layer "B.Cu") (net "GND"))
 (segment (start 194.33 80.58) (end 194.5 80.75) (width 0.2) (layer "F.Cu") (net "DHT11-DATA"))
 (segment (start 168.46 45) (end 168.46 47.65) (width 0.2) (layer "F.Cu") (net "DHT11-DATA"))
 (segment (start 194.33 78.27) (end 194.33 80.58) (width 0.2) (layer "F.Cu") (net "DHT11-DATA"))
 (segment (start 168.46 47.65) (end 171.31 50.5) (width 0.2) (layer "F.Cu") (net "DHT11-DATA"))
 (via (at 194.5 80.75) (size 0.6) (drill 0.3) (layers "F.Cu" "B.Cu") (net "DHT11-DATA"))
 (segment (start 171.31 54.06) (end 171.31 50.5) (width 0.2) (layer "B.Cu") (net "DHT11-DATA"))
 (segment (start 194.5 80.75) (end 194.5 77.25) (width 0.2) (layer "B.Cu") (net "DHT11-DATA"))
 (segment (start 194.5 77.25) (end 171.31 54.06) (width 0.2) (layer "B.Cu") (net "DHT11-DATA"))
 (segment (start 189.25 78.27) (end 189.25 80) (width 0.2) (layer "F.Cu") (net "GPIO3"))
 (segment (start 189.25 80) (end 187.75 81.5) (width 0.2) (layer "F.Cu") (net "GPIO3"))
 (via (at 187.75 81.5) (size 0.6) (drill 0.3) (layers "F.Cu" "B.Cu") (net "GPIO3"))
 (segment (start 179.5 80.75) (end 179.5 77.25) (width 0.2) (layer "B.Cu") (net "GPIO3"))
 (segment (start 156.75 51.38) (end 149.54 44.17) (width 0.2) (layer "B.Cu") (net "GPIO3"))
 (segment (start 187.75 81.5) (end 180.25 81.5) (width 0.2) (layer "B.Cu") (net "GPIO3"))
 (segment (start 180.25 81.5) (end 179.5 80.75) (width 0.2) (layer "B.Cu") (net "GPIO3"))
 (segment (start 175 72.75) (end 156.75 72.75) (width 0.2) (layer "B.Cu") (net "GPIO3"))
 (segment (start 179.5 77.25) (end 175 72.75) (width 0.2) (layer "B.Cu") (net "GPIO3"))
 (segment (start 156.75 72.75) (end 156.75 51.38) (width 0.2) (layer "B.Cu") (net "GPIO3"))
 (segment (start 191.79 79.54) (end 193.25 81) (width 0.2) (layer "F.Cu") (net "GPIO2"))
 (segment (start 191.79 78.27) (end 191.79 79.54) (width 0.2) (layer "F.Cu") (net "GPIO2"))
 (via (at 193.25 81) (size 0.6) (drill 0.3) (layers "F.Cu" "B.Cu") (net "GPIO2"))
 (segment (start 193.25 81) (end 193.25 78.25) (width 0.2) (layer "B.Cu") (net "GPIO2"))
 (segment (start 193.25 78.25) (end 171.92 56.92) (width 0.2) (layer "B.Cu") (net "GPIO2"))
 (segment (start 171.92 56.92) (end 170.04 56.92) (width 0.2) (layer "B.Cu") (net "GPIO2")))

